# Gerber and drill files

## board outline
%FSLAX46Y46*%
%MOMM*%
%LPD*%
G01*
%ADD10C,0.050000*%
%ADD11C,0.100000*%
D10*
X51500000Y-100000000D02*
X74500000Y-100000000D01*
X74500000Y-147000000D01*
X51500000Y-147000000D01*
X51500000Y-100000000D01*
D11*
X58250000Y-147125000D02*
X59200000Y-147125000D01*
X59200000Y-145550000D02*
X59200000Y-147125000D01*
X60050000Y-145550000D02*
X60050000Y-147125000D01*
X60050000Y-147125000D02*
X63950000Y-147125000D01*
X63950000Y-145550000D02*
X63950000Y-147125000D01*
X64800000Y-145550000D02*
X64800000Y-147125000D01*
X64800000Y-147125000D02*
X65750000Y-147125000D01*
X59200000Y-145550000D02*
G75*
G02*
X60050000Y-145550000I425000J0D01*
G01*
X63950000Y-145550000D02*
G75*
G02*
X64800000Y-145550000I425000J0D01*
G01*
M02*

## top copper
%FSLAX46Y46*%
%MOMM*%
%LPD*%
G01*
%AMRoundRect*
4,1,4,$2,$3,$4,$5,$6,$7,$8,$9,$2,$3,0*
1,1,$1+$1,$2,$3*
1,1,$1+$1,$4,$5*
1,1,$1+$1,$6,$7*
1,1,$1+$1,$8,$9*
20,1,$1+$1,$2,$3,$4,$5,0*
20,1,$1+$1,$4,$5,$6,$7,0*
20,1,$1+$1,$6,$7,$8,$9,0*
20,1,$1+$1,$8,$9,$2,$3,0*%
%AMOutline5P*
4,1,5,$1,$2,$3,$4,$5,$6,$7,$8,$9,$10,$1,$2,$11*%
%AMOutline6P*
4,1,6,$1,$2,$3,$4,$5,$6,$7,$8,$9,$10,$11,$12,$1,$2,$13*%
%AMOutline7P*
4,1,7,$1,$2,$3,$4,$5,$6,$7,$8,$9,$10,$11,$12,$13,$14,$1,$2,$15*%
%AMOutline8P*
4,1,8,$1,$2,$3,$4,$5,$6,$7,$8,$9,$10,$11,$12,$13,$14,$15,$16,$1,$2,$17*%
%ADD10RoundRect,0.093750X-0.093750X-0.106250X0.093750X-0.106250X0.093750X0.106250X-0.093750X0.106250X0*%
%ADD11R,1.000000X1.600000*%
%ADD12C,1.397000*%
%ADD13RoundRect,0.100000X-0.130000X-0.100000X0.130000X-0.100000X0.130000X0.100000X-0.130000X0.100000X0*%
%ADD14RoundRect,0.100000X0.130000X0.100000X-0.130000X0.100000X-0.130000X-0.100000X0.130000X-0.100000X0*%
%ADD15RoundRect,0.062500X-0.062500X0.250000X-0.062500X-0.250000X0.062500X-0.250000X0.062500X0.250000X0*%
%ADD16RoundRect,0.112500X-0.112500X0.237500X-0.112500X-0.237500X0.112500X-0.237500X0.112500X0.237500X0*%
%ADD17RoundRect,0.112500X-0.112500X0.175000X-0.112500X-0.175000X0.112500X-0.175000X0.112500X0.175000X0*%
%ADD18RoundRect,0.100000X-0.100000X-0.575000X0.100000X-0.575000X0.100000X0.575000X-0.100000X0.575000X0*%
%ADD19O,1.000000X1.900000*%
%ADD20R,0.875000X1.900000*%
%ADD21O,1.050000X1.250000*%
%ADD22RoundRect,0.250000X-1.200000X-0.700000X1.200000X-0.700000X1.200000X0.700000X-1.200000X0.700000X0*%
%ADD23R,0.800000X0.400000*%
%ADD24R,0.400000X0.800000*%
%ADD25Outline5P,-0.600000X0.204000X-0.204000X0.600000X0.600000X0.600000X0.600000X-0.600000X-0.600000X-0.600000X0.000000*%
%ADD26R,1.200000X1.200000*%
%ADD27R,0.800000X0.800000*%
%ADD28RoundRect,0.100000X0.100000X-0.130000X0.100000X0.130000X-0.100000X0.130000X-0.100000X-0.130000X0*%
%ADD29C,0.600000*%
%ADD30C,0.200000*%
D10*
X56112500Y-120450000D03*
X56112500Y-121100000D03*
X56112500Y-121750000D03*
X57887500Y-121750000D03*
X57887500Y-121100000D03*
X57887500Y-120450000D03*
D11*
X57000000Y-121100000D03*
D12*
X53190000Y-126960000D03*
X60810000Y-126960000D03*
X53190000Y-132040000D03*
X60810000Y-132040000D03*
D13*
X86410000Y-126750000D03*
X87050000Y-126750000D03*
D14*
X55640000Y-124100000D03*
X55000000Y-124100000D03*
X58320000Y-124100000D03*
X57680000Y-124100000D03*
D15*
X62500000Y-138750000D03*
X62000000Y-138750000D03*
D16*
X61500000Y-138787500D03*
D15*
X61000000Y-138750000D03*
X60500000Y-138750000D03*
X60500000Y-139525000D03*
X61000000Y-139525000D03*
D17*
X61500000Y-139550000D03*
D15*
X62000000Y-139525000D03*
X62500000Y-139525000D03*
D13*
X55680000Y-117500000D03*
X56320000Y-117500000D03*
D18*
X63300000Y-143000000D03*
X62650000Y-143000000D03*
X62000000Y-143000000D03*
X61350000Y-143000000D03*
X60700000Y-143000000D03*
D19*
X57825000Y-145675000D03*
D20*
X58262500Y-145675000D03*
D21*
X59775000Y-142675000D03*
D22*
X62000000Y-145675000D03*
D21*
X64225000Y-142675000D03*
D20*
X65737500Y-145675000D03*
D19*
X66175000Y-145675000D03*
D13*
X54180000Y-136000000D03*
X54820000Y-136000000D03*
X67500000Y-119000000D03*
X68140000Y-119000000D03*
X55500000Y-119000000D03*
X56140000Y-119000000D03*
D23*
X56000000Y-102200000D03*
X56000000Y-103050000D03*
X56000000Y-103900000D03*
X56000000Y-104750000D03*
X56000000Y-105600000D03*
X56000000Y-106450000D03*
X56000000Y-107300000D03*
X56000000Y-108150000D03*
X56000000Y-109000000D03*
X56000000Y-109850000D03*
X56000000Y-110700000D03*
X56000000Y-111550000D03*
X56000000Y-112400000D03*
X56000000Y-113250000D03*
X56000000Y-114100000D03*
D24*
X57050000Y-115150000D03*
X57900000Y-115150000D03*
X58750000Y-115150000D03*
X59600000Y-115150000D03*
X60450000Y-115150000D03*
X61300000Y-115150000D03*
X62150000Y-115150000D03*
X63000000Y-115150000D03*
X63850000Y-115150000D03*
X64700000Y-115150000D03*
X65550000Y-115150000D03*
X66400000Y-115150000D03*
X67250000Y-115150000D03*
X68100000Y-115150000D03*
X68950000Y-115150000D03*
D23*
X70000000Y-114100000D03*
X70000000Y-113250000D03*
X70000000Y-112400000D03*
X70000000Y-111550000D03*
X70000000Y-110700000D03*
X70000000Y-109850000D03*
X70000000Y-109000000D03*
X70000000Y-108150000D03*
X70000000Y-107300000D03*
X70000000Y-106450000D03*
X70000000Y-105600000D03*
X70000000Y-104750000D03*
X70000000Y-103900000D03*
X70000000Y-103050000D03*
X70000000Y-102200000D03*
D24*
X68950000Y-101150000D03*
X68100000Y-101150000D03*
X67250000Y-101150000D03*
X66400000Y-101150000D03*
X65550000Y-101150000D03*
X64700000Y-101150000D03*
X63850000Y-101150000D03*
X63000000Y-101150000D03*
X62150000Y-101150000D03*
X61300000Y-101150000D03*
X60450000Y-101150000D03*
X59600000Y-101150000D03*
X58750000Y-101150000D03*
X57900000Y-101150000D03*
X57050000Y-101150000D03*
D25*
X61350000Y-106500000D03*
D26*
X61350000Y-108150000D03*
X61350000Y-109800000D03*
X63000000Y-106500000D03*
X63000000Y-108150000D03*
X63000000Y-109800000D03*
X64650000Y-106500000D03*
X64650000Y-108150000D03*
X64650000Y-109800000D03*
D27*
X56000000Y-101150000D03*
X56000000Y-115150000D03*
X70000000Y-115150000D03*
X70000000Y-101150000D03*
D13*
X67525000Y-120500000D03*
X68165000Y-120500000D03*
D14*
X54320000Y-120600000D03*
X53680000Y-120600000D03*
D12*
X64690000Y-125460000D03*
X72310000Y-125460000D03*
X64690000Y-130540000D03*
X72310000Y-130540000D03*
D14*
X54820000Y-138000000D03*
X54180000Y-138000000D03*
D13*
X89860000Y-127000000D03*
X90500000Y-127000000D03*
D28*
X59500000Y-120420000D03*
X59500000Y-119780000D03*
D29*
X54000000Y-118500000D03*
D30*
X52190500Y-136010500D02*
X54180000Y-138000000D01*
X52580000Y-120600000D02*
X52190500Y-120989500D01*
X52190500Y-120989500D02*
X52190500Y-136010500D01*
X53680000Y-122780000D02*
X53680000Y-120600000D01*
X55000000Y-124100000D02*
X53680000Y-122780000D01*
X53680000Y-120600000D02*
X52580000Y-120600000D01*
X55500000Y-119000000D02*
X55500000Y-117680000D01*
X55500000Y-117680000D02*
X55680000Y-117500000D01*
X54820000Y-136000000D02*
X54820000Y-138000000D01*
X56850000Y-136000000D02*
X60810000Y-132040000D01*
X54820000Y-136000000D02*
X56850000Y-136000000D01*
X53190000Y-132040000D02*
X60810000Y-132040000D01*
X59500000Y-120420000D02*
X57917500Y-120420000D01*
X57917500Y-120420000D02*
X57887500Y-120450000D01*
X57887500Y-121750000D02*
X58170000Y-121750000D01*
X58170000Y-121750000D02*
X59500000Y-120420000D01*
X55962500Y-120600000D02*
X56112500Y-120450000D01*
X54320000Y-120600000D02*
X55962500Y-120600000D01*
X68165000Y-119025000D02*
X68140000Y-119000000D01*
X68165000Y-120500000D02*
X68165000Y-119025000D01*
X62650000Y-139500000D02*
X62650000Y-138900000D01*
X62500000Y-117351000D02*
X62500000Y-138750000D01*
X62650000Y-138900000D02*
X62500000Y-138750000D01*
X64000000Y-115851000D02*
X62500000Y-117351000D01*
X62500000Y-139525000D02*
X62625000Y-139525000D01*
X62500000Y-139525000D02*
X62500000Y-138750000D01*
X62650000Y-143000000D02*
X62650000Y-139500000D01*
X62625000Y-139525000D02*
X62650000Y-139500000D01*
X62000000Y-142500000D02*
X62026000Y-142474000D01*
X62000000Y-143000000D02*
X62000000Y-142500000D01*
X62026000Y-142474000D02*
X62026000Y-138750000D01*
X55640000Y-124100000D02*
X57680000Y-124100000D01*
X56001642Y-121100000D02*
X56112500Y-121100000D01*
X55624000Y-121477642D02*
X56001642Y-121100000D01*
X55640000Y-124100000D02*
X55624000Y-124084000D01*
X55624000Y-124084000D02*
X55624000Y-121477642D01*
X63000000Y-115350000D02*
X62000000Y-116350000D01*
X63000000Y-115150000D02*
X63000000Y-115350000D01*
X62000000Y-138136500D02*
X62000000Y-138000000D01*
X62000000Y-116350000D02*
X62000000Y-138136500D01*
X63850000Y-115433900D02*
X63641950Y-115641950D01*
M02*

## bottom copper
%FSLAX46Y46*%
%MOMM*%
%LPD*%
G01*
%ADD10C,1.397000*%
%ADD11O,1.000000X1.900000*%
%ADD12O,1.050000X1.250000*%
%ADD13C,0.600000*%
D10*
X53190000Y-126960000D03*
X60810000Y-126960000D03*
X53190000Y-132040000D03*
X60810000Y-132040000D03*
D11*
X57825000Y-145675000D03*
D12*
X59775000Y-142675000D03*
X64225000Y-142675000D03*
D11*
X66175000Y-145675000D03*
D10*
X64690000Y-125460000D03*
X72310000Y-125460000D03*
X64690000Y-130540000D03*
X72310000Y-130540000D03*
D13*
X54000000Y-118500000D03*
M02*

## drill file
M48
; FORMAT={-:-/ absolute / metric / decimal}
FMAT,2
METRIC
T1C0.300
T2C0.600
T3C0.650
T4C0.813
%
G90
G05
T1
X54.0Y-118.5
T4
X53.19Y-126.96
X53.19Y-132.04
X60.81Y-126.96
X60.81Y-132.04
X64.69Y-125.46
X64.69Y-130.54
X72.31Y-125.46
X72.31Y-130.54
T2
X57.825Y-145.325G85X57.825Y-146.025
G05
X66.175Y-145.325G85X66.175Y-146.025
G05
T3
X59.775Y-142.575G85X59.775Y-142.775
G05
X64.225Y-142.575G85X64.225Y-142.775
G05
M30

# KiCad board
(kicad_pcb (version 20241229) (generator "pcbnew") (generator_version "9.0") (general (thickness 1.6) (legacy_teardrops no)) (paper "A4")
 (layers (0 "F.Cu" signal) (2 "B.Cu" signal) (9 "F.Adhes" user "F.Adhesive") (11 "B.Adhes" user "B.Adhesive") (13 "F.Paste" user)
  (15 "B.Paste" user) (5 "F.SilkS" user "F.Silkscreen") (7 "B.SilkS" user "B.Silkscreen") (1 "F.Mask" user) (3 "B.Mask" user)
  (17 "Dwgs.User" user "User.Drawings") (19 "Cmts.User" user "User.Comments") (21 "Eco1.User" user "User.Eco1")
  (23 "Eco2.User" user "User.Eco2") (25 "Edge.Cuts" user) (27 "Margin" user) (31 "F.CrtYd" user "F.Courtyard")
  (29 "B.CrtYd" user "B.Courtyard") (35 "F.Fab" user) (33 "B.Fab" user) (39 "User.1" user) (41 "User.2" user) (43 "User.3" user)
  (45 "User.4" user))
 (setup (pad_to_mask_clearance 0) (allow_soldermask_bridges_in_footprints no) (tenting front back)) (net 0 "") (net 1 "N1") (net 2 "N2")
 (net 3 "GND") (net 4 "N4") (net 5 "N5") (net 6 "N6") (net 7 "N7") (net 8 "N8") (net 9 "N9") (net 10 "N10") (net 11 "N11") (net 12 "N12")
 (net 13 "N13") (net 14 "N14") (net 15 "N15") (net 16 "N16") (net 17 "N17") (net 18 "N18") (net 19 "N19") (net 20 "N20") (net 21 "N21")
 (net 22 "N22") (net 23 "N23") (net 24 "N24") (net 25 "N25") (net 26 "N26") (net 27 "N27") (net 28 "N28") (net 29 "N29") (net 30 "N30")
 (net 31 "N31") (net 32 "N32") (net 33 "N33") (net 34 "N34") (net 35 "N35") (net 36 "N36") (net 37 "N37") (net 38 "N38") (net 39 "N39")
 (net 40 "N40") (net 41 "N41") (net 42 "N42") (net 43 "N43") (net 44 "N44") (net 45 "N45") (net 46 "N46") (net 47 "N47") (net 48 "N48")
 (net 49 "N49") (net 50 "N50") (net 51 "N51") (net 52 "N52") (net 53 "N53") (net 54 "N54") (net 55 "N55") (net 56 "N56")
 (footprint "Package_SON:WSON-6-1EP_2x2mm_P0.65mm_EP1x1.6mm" (layer "F.Cu") (at 57 121.1)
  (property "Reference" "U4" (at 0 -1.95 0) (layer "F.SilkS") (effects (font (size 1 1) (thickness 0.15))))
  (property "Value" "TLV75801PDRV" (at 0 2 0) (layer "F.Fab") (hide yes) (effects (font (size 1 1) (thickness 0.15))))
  (pad "" smd roundrect (at 0 -0.4) (size 0.81 0.64) (layers "F.Paste") (roundrect_rratio 0.25))
  (pad "" smd roundrect (at 0 0.4) (size 0.81 0.64) (layers "F.Paste") (roundrect_rratio 0.25))
  (pad "1" smd roundrect (at -0.8875 -0.65) (size 0.375 0.4) (layers "F.Cu" "F.Mask" "F.Paste") (roundrect_rratio 0.25) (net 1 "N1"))
  (pad "2" smd roundrect (at -0.8875 0) (size 0.375 0.4) (layers "F.Cu" "F.Mask" "F.Paste") (roundrect_rratio 0.25) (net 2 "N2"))
  (pad "3" smd roundrect (at -0.8875 0.65) (size 0.375 0.4) (layers "F.Cu" "F.Mask" "F.Paste") (roundrect_rratio 0.25) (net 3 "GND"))
  (pad "4" smd roundrect (at 0.8875 0.65) (size 0.375 0.4) (layers "F.Cu" "F.Mask" "F.Paste") (roundrect_rratio 0.25) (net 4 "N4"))
  (pad "5" smd roundrect (at 0.8875 0) (size 0.375 0.4) (layers "F.Cu" "F.Mask" "F.Paste") (roundrect_rratio 0.25) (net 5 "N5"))
  (pad "6" smd roundrect (at 0.8875 -0.65) (size 0.375 0.4) (layers "F.Cu" "F.Mask" "F.Paste") (roundrect_rratio 0.25) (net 4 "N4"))
  (pad "7" smd rect (at 0 0) (size 1 1.6) (layers "F.Cu" "F.Mask") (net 3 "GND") (zone_connect 2)))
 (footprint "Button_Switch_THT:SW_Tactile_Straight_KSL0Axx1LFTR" (layer "F.Cu") (at 53.19 126.96)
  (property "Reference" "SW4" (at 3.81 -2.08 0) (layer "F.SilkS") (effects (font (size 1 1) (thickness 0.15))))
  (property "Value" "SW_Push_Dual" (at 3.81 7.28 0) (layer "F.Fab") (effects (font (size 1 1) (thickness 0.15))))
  (pad "1" thru_hole circle (at 0 0) (size 1.397 1.397) (drill 0.8128) (layers "*.Cu" "*.Mask") (remove_unused_layers no) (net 3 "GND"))
  (pad "1" thru_hole circle (at 7.62 0) (size 1.397 1.397) (drill 0.8128) (layers "*.Cu" "*.Mask") (remove_unused_layers no) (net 3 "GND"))
  (pad "2" thru_hole circle (at 0 5.08) (size 1.397 1.397) (drill 0.8128) (layers "*.Cu" "*.Mask") (remove_unused_layers no) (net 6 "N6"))
  (pad "2" thru_hole circle (at 7.62 5.08) (size 1.397 1.397) (drill 0.8128) (layers "*.Cu" "*.Mask") (remove_unused_layers no) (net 6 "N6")))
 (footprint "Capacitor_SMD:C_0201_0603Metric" (layer "F.Cu") (at 86.73 126.75)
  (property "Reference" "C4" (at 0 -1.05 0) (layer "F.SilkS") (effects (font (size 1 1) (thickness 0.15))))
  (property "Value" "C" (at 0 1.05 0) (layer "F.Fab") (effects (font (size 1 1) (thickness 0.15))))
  (pad "" smd roundrect (at -0.345 0) (size 0.318 0.36) (layers "F.Paste") (roundrect_rratio 0.25))
  (pad "" smd roundrect (at 0.345 0) (size 0.318 0.36) (layers "F.Paste") (roundrect_rratio 0.25))
  (pad "1" smd roundrect (at -0.32 0) (size 0.46 0.4) (layers "F.Cu" "F.Mask") (roundrect_rratio 0.25) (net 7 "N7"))
  (pad "2" smd roundrect (at 0.32 0) (size 0.46 0.4) (layers "F.Cu" "F.Mask") (roundrect_rratio 0.25) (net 3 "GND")))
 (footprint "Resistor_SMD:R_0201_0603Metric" (layer "F.Cu") (at 55.32 124.1 180)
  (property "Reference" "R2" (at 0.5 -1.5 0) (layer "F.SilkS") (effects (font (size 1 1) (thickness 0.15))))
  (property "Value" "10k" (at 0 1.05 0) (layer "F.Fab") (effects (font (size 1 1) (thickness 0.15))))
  (pad "" smd roundrect (at -0.345 0 180) (size 0.318 0.36) (layers "F.Paste") (roundrect_rratio 0.25))
  (pad "" smd roundrect (at 0.345 0 180) (size 0.318 0.36) (layers "F.Paste") (roundrect_rratio 0.25))
  (pad "1" smd roundrect (at -0.32 0 180) (size 0.46 0.4) (layers "F.Cu" "F.Mask") (roundrect_rratio 0.25) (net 2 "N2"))
  (pad "2" smd roundrect (at 0.32 0 180) (size 0.46 0.4) (layers "F.Cu" "F.Mask") (roundrect_rratio 0.25) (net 3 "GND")))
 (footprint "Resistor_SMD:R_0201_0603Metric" (layer "F.Cu") (at 58 124.1 180)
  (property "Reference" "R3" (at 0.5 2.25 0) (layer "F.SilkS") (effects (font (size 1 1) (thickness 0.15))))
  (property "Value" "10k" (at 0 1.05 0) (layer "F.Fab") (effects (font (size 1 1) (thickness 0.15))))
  (pad "" smd roundrect (at -0.345 0 180) (size 0.318 0.36) (layers "F.Paste") (roundrect_rratio 0.25))
  (pad "" smd roundrect (at 0.345 0 180) (size 0.318 0.36) (layers "F.Paste") (roundrect_rratio 0.25))
  (pad "1" smd roundrect (at -0.32 0 180) (size 0.46 0.4) (layers "F.Cu" "F.Mask") (roundrect_rratio 0.25) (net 1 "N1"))
  (pad "2" smd roundrect (at 0.32 0 180) (size 0.46 0.4) (layers "F.Cu" "F.Mask") (roundrect_rratio 0.25) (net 2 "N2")))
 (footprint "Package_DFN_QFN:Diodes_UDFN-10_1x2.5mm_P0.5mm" (layer "F.Cu") (at 61.5 139.1375 -90)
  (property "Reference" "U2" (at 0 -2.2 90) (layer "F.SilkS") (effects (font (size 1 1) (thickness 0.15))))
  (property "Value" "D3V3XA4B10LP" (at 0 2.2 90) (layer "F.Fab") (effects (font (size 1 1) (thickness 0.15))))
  (pad "1" smd roundrect (at -0.3875 -1 270) (size 0.625 0.25) (layers "F.Cu" "F.Mask" "F.Paste") (roundrect_rratio 0.25) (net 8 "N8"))
  (pad "2" smd roundrect (at -0.3875 -0.5 270) (size 0.625 0.25) (layers "F.Cu" "F.Mask" "F.Paste") (roundrect_rratio 0.25) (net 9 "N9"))
  (pad "3" smd roundrect (at -0.35 0 270) (size 0.7 0.45) (layers "F.Cu" "F.Mask" "F.Paste") (roundrect_rratio 0.25) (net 3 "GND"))
  (pad "4" smd roundrect (at -0.3875 0.5 270) (size 0.625 0.25) (layers "F.Cu" "F.Mask" "F.Paste") (roundrect_rratio 0.25) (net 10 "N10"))
  (pad "5" smd roundrect (at -0.3875 1 270) (size 0.625 0.25) (layers "F.Cu" "F.Mask" "F.Paste") (roundrect_rratio 0.25) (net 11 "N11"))
  (pad "6" smd roundrect (at 0.3875 1 270) (size 0.625 0.25) (layers "F.Cu" "F.Mask" "F.Paste") (roundrect_rratio 0.25) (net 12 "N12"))
  (pad "7" smd roundrect (at 0.3875 0.5 270) (size 0.625 0.25) (layers "F.Cu" "F.Mask" "F.Paste") (roundrect_rratio 0.25) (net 10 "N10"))
  (pad "8" smd roundrect (at 0.4125 0 270) (size 0.575 0.45) (layers "F.Cu" "F.Mask" "F.Paste") (roundrect_rratio 0.25) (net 3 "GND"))
  (pad "9" smd roundrect (at 0.3875 -0.5 270) (size 0.625 0.25) (layers "F.Cu" "F.Mask" "F.Paste") (roundrect_rratio 0.25) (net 9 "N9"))
  (pad "10" smd roundrect (at 0.3875 -1 270) (size 0.625 0.25) (layers "F.Cu" "F.Mask" "F.Paste") (roundrect_rratio 0.25) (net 8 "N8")))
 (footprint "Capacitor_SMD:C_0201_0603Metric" (layer "F.Cu") (at 56 117.5)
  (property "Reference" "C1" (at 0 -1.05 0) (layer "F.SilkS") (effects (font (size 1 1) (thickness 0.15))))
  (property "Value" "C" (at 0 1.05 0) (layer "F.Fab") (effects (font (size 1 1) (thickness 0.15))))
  (pad "" smd roundrect (at -0.345 0) (size 0.318 0.36) (layers "F.Paste") (roundrect_rratio 0.25))
  (pad "" smd roundrect (at 0.345 0) (size 0.318 0.36) (layers "F.Paste") (roundrect_rratio 0.25))
  (pad "1" smd roundrect (at -0.32 0) (size 0.46 0.4) (layers "F.Cu" "F.Mask") (roundrect_rratio 0.25) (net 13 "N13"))
  (pad "2" smd roundrect (at 0.32 0) (size 0.46 0.4) (layers "F.Cu" "F.Mask") (roundrect_rratio 0.25) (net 3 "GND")))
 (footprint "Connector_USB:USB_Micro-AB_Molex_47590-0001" (layer "F.Cu") (at 62 146.025)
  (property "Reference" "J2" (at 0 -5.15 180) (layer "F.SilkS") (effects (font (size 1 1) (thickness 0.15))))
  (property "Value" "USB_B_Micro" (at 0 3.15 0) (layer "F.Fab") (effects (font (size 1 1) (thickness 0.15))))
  (fp_line (start -3.75 1.1) (end -2.8 1.1) (stroke (width 0.1) (type solid)) (layer "Edge.Cuts"))
  (fp_line (start -2.8 -0.475) (end -2.8 1.1) (stroke (width 0.1) (type solid)) (layer "Edge.Cuts"))
  (fp_line (start -1.95 -0.475) (end -1.95 1.1) (stroke (width 0.1) (type solid)) (layer "Edge.Cuts"))
  (fp_line (start -1.95 1.1) (end 1.95 1.1) (stroke (width 0.1) (type solid)) (layer "Edge.Cuts"))
  (fp_line (start 1.95 -0.475) (end 1.95 1.1) (stroke (width 0.1) (type solid)) (layer "Edge.Cuts"))
  (fp_line (start 2.8 -0.475) (end 2.8 1.1) (stroke (width 0.1) (type solid)) (layer "Edge.Cuts"))
  (fp_line (start 2.8 1.1) (end 3.75 1.1) (stroke (width 0.1) (type solid)) (layer "Edge.Cuts"))
  (fp_arc (start -2.8 -0.475) (mid -2.375 -0.9) (end -1.95 -0.475) (stroke (width 0.1) (type solid)) (layer "Edge.Cuts"))
  (fp_arc (start 1.95 -0.475) (mid 2.375 -0.9) (end 2.8 -0.475) (stroke (width 0.1) (type solid)) (layer "Edge.Cuts"))
  (pad "" smd rect (at -3.5 -0.35) (size 0.3 0.85) (layers "F.Paste"))
  (pad "" smd rect (at 3.5 -0.35) (size 0.3 0.85) (layers "F.Paste"))
  (pad "1" smd roundrect (at 1.3 -3.025) (size 0.4 1.35) (layers "F.Cu" "F.Mask" "F.Paste") (roundrect_rratio 0.25) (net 10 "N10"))
  (pad "2" smd roundrect (at 0.65 -3.025) (size 0.4 1.35) (layers "F.Cu" "F.Mask" "F.Paste") (roundrect_rratio 0.25) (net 8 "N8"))
  (pad "3" smd roundrect (at 0 -3.025) (size 0.4 1.35) (layers "F.Cu" "F.Mask" "F.Paste") (roundrect_rratio 0.25) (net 9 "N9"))
  (pad "4" smd roundrect (at -0.65 -3.025) (size 0.4 1.35) (layers "F.Cu" "F.Mask" "F.Paste") (roundrect_rratio 0.25) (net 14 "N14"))
  (pad "5" smd roundrect (at -1.3 -3.025) (size 0.4 1.35) (layers "F.Cu" "F.Mask" "F.Paste") (roundrect_rratio 0.25) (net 3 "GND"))
  (pad "6" thru_hole oval (at -4.175 -0.35) (size 1 1.9) (drill oval 0.6 1.3) (layers "*.Cu" "*.Mask") (remove_unused_layers no)
   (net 3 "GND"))
  (pad "6" smd rect (at -3.7375 -0.35) (size 0.875 1.9) (layers "F.Cu" "F.Mask") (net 3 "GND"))
  (pad "6" thru_hole oval (at -2.225 -3.35) (size 1.05 1.25) (drill oval 0.65 0.85) (layers "*.Cu" "*.Mask") (remove_unused_layers no)
   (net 3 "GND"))
  (pad "6" smd roundrect (at 0 -0.35) (size 2.9 1.9) (layers "F.Cu" "F.Mask" "F.Paste") (roundrect_rratio 0.1315789474) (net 3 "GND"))
  (pad "6" thru_hole oval (at 2.225 -3.35) (size 1.05 1.25) (drill oval 0.65 0.85) (layers "*.Cu" "*.Mask") (remove_unused_layers no)
   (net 3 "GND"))
  (pad "6" smd rect (at 3.7375 -0.35) (size 0.875 1.9) (layers "F.Cu" "F.Mask") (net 3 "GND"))
  (pad "6" thru_hole oval (at 4.175 -0.35) (size 1 1.9) (drill oval 0.6 1.3) (layers "*.Cu" "*.Mask") (remove_unused_layers no)
   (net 3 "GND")))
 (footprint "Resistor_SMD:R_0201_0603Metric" (layer "F.Cu") (at 54.5 136)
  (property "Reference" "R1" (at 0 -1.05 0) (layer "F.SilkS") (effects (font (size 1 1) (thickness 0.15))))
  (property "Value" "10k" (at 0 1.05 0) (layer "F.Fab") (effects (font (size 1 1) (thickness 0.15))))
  (pad "" smd roundrect (at -0.345 0) (size 0.318 0.36) (layers "F.Paste") (roundrect_rratio 0.25))
  (pad "" smd roundrect (at 0.345 0) (size 0.318 0.36) (layers "F.Paste") (roundrect_rratio 0.25))
  (pad "1" smd roundrect (at -0.32 0) (size 0.46 0.4) (layers "F.Cu" "F.Mask") (roundrect_rratio 0.25) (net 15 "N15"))
  (pad "2" smd roundrect (at 0.32 0) (size 0.46 0.4) (layers "F.Cu" "F.Mask") (roundrect_rratio 0.25) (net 6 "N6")))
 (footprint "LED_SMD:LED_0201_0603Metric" (layer "F.Cu") (at 67.82 119)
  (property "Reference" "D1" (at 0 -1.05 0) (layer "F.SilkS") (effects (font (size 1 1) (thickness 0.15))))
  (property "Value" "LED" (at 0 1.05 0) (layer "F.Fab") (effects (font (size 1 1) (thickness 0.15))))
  (pad "" smd roundrect (at -0.345 0) (size 0.318 0.36) (layers "F.Paste") (roundrect_rratio 0.25))
  (pad "" smd roundrect (at 0.345 0) (size 0.318 0.36) (layers "F.Paste") (roundrect_rratio 0.25))
  (pad "1" smd roundrect (at -0.32 0) (size 0.46 0.4) (layers "F.Cu" "F.Mask") (roundrect_rratio 0.25) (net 3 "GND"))
  (pad "2" smd roundrect (at 0.32 0) (size 0.46 0.4) (layers "F.Cu" "F.Mask") (roundrect_rratio 0.25) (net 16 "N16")))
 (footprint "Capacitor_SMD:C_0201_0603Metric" (layer "F.Cu") (at 55.82 119)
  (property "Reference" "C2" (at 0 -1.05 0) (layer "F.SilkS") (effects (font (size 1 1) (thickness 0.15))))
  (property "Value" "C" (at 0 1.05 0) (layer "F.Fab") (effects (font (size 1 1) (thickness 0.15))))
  (pad "" smd roundrect (at -0.345 0) (size 0.318 0.36) (layers "F.Paste") (roundrect_rratio 0.25))
  (pad "" smd roundrect (at 0.345 0) (size 0.318 0.36) (layers "F.Paste") (roundrect_rratio 0.25))
  (pad "1" smd roundrect (at -0.32 0) (size 0.46 0.4) (layers "F.Cu" "F.Mask") (roundrect_rratio 0.25) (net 13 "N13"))
  (pad "2" smd roundrect (at 0.32 0) (size 0.46 0.4) (layers "F.Cu" "F.Mask") (roundrect_rratio 0.25) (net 3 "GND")))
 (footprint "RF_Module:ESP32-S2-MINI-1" (layer "F.Cu") (at 63 105.6)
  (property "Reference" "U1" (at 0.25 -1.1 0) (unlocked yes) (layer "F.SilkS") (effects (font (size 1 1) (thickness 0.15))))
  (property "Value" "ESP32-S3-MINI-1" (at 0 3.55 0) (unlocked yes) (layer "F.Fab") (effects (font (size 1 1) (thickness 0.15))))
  (pad "1" smd rect (at -7 -3.4) (size 0.8 0.4) (layers "F.Cu" "F.Mask" "F.Paste") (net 3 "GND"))
  (pad "2" smd rect (at -7 -2.55) (size 0.8 0.4) (layers "F.Cu" "F.Mask" "F.Paste") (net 3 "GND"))
  (pad "3" smd rect (at -7 -1.7) (size 0.8 0.4) (layers "F.Cu" "F.Mask" "F.Paste") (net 13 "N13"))
  (pad "4" smd rect (at -7 -0.85) (size 0.8 0.4) (layers "F.Cu" "F.Mask" "F.Paste") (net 7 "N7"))
  (pad "5" smd rect (at -7 0) (size 0.8 0.4) (layers "F.Cu" "F.Mask" "F.Paste") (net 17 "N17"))
  (pad "6" smd rect (at -7 0.85) (size 0.8 0.4) (layers "F.Cu" "F.Mask" "F.Paste") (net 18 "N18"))
  (pad "7" smd rect (at -7 1.7) (size 0.8 0.4) (layers "F.Cu" "F.Mask" "F.Paste") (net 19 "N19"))
  (pad "8" smd rect (at -7 2.55) (size 0.8 0.4) (layers "F.Cu" "F.Mask" "F.Paste") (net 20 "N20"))
  (pad "9" smd rect (at -7 3.4) (size 0.8 0.4) (layers "F.Cu" "F.Mask" "F.Paste") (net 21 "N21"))
  (pad "10" smd rect (at -7 4.25) (size 0.8 0.4) (layers "F.Cu" "F.Mask" "F.Paste") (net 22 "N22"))
  (pad "11" smd rect (at -7 5.1) (size 0.8 0.4) (layers "F.Cu" "F.Mask" "F.Paste") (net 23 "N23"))
  (pad "12" smd rect (at -7 5.95) (size 0.8 0.4) (layers "F.Cu" "F.Mask" "F.Paste") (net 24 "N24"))
  (pad "13" smd rect (at -7 6.8) (size 0.8 0.4) (layers "F.Cu" "F.Mask" "F.Paste") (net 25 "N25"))
  (pad "14" smd rect (at -7 7.65) (size 0.8 0.4) (layers "F.Cu" "F.Mask" "F.Paste") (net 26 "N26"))
  (pad "15" smd rect (at -7 8.5) (size 0.8 0.4) (layers "F.Cu" "F.Mask" "F.Paste") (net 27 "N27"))
  (pad "16" smd rect (at -5.95 9.55 90) (size 0.8 0.4) (layers "F.Cu" "F.Mask" "F.Paste") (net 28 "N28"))
  (pad "17" smd rect (at -5.1 9.55 90) (size 0.8 0.4) (layers "F.Cu" "F.Mask" "F.Paste") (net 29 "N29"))
  (pad "18" smd rect (at -4.25 9.55 90) (size 0.8 0.4) (layers "F.Cu" "F.Mask" "F.Paste") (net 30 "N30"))
  (pad "19" smd rect (at -3.4 9.55 90) (size 0.8 0.4) (layers "F.Cu" "F.Mask" "F.Paste") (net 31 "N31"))
  (pad "20" smd rect (at -2.55 9.55 90) (size 0.8 0.4) (layers "F.Cu" "F.Mask" "F.Paste") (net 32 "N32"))
  (pad "21" smd rect (at -1.7 9.55 90) (size 0.8 0.4) (layers "F.Cu" "F.Mask" "F.Paste") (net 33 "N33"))
  (pad "22" smd rect (at -0.85 9.55 90) (size 0.8 0.4) (layers "F.Cu" "F.Mask" "F.Paste") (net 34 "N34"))
  (pad "23" smd rect (at 0 9.55 90) (size 0.8 0.4) (layers "F.Cu" "F.Mask" "F.Paste") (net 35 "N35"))
  (pad "24" smd rect (at 0.85 9.55 90) (size 0.8 0.4) (layers "F.Cu" "F.Mask" "F.Paste") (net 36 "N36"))
  (pad "25" smd rect (at 1.7 9.55 90) (size 0.8 0.4) (layers "F.Cu" "F.Mask" "F.Paste") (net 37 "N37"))
  (pad "26" smd rect (at 2.55 9.55 90) (size 0.8 0.4) (layers "F.Cu" "F.Mask" "F.Paste") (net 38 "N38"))
  (pad "27" smd rect (at 3.4 9.55 90) (size 0.8 0.4) (layers "F.Cu" "F.Mask" "F.Paste") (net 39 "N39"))
  (pad "28" smd rect (at 4.25 9.55 90) (size 0.8 0.4) (layers "F.Cu" "F.Mask" "F.Paste") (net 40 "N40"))
  (pad "29" smd rect (at 5.1 9.55 90) (size 0.8 0.4) (layers "F.Cu" "F.Mask" "F.Paste") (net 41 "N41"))
  (pad "30" smd rect (at 5.95 9.55 90) (size 0.8 0.4) (layers "F.Cu" "F.Mask" "F.Paste") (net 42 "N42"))
  (pad "31" smd rect (at 7 8.5) (size 0.8 0.4) (layers "F.Cu" "F.Mask" "F.Paste") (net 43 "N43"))
  (pad "32" smd rect (at 7 7.65) (size 0.8 0.4) (layers "F.Cu" "F.Mask" "F.Paste") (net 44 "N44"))
  (pad "33" smd rect (at 7 6.8) (size 0.8 0.4) (layers "F.Cu" "F.Mask" "F.Paste") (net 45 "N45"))
  (pad "34" smd rect (at 7 5.95) (size 0.8 0.4) (layers "F.Cu" "F.Mask" "F.Paste") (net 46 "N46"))
  (pad "35" smd rect (at 7 5.1) (size 0.8 0.4) (layers "F.Cu" "F.Mask" "F.Paste") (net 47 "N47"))
  (pad "36" smd rect (at 7 4.25) (size 0.8 0.4) (layers "F.Cu" "F.Mask" "F.Paste") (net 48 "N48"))
  (pad "37" smd rect (at 7 3.4) (size 0.8 0.4) (layers "F.Cu" "F.Mask" "F.Paste") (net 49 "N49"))
  (pad "38" smd rect (at 7 2.55) (size 0.8 0.4) (layers "F.Cu" "F.Mask" "F.Paste") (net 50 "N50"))
  (pad "39" smd rect (at 7 1.7) (size 0.8 0.4) (layers "F.Cu" "F.Mask" "F.Paste") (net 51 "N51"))
  (pad "40" smd rect (at 7 0.85) (size 0.8 0.4) (layers "F.Cu" "F.Mask" "F.Paste") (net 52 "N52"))
  (pad "41" smd rect (at 7 0) (size 0.8 0.4) (layers "F.Cu" "F.Mask" "F.Paste") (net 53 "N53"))
  (pad "42" smd rect (at 7 -0.85) (size 0.8 0.4) (layers "F.Cu" "F.Mask" "F.Paste") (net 3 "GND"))
  (pad "43" smd rect (at 7 -1.7) (size 0.8 0.4) (layers "F.Cu" "F.Mask" "F.Paste") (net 3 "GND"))
  (pad "44" smd rect (at 7 -2.55) (size 0.8 0.4) (layers "F.Cu" "F.Mask" "F.Paste") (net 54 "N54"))
  (pad "45" smd rect (at 7 -3.4) (size 0.8 0.4) (layers "F.Cu" "F.Mask" "F.Paste") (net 6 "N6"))
  (pad "46" smd rect (at 5.95 -4.45 90) (size 0.8 0.4) (layers "F.Cu" "F.Mask" "F.Paste") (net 3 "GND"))
  (pad "47" smd rect (at 5.1 -4.45 90) (size 0.8 0.4) (layers "F.Cu" "F.Mask" "F.Paste") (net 3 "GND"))
  (pad "48" smd rect (at 4.25 -4.45 90) (size 0.8 0.4) (layers "F.Cu" "F.Mask" "F.Paste") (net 3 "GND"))
  (pad "49" smd rect (at 3.4 -4.45 90) (size 0.8 0.4) (layers "F.Cu" "F.Mask" "F.Paste") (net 3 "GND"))
  (pad "50" smd rect (at 2.55 -4.45 90) (size 0.8 0.4) (layers "F.Cu" "F.Mask" "F.Paste") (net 3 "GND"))
  (pad "51" smd rect (at 1.7 -4.45 90) (size 0.8 0.4) (layers "F.Cu" "F.Mask" "F.Paste") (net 3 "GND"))
  (pad "52" smd rect (at 0.85 -4.45 90) (size 0.8 0.4) (layers "F.Cu" "F.Mask" "F.Paste") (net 3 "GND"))
  (pad "53" smd rect (at 0 -4.45 90) (size 0.8 0.4) (layers "F.Cu" "F.Mask" "F.Paste") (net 3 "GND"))
  (pad "54" smd rect (at -0.85 -4.45 90) (size 0.8 0.4) (layers "F.Cu" "F.Mask" "F.Paste") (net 3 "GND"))
  (pad "55" smd rect (at -1.7 -4.45 90) (size 0.8 0.4) (layers "F.Cu" "F.Mask" "F.Paste") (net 3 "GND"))
  (pad "56" smd rect (at -2.55 -4.45 90) (size 0.8 0.4) (layers "F.Cu" "F.Mask" "F.Paste") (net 3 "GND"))
  (pad "57" smd rect (at -3.4 -4.45 90) (size 0.8 0.4) (layers "F.Cu" "F.Mask" "F.Paste") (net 3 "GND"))
  (pad "58" smd rect (at -4.25 -4.45 90) (size 0.8 0.4) (layers "F.Cu" "F.Mask" "F.Paste") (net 3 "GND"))
  (pad "59" smd rect (at -5.1 -4.45 90) (size 0.8 0.4) (layers "F.Cu" "F.Mask" "F.Paste") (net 3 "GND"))
  (pad "60" smd rect (at -5.95 -4.45 90) (size 0.8 0.4) (layers "F.Cu" "F.Mask" "F.Paste") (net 3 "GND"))
  (pad "61" smd roundrect (at -1.65 0.9) (size 1.2 1.2) (layers "F.Cu" "F.Mask" "F.Paste") (roundrect_rratio 0) (chamfer_ratio 0.33)
   (chamfer top_left) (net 3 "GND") (zone_connect 2))
  (pad "61" smd rect (at -1.65 2.55) (size 1.2 1.2) (layers "F.Cu" "F.Mask" "F.Paste") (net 3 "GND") (zone_connect 2))
  (pad "61" smd rect (at -1.65 4.2) (size 1.2 1.2) (layers "F.Cu" "F.Mask" "F.Paste") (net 3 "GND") (zone_connect 2))
  (pad "61" smd rect (at 0 0.9) (size 1.2 1.2) (layers "F.Cu" "F.Mask" "F.Paste") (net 3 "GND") (zone_connect 2))
  (pad "61" smd rect (at 0 2.55) (size 1.2 1.2) (layers "F.Cu" "F.Mask" "F.Paste") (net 3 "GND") (zone_connect 2))
  (pad "61" smd rect (at 0 4.2) (size 1.2 1.2) (layers "F.Cu" "F.Mask" "F.Paste") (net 3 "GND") (zone_connect 2))
  (pad "61" smd rect (at 1.65 0.9) (size 1.2 1.2) (layers "F.Cu" "F.Mask" "F.Paste") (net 3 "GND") (zone_connect 2))
  (pad "61" smd rect (at 1.65 2.55) (size 1.2 1.2) (layers "F.Cu" "F.Mask" "F.Paste") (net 3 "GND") (zone_connect 2))
  (pad "61" smd rect (at 1.65 4.2) (size 1.2 1.2) (layers "F.Cu" "F.Mask" "F.Paste") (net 3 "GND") (zone_connect 2))
  (pad "62" smd rect (at -7 -4.45) (size 0.8 0.8) (layers "F.Cu" "F.Mask" "F.Paste") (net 3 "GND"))
  (pad "63" smd rect (at -7 9.55) (size 0.8 0.8) (layers "F.Cu" "F.Mask" "F.Paste") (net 3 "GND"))
  (pad "64" smd rect (at 7 9.55) (size 0.8 0.8) (layers "F.Cu" "F.Mask" "F.Paste") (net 3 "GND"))
  (pad "65" smd rect (at 7 -4.45) (size 0.8 0.8) (layers "F.Cu" "F.Mask" "F.Paste") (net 3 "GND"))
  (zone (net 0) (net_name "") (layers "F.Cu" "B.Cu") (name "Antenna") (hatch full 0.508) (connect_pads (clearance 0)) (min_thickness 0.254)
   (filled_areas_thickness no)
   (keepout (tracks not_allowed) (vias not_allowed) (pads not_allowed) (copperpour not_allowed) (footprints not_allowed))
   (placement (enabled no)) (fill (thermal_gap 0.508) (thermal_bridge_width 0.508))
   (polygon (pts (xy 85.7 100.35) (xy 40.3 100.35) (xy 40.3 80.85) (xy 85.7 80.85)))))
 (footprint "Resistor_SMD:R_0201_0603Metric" (layer "F.Cu") (at 67.845 120.5)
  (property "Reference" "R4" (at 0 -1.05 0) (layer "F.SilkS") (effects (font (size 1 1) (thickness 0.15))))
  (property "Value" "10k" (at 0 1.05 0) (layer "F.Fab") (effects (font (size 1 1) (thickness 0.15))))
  (pad "" smd roundrect (at -0.345 0) (size 0.318 0.36) (layers "F.Paste") (roundrect_rratio 0.25))
  (pad "" smd roundrect (at 0.345 0) (size 0.318 0.36) (layers "F.Paste") (roundrect_rratio 0.25))
  (pad "1" smd roundrect (at -0.32 0) (size 0.46 0.4) (layers "F.Cu" "F.Mask") (roundrect_rratio 0.25) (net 1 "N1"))
  (pad "2" smd roundrect (at 0.32 0) (size 0.46 0.4) (layers "F.Cu" "F.Mask") (roundrect_rratio 0.25) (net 16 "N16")))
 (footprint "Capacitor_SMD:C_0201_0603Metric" (layer "F.Cu") (at 54 120.6 180)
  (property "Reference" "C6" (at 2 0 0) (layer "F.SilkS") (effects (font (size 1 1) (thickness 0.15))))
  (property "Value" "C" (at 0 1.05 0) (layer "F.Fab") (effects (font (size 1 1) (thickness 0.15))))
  (pad "" smd roundrect (at -0.345 0 180) (size 0.318 0.36) (layers "F.Paste") (roundrect_rratio 0.25))
  (pad "" smd roundrect (at 0.345 0 180) (size 0.318 0.36) (layers "F.Paste") (roundrect_rratio 0.25))
  (pad "1" smd roundrect (at -0.32 0 180) (size 0.46 0.4) (layers "F.Cu" "F.Mask") (roundrect_rratio 0.25) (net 1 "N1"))
  (pad "2" smd roundrect (at 0.32 0 180) (size 0.46 0.4) (layers "F.Cu" "F.Mask") (roundrect_rratio 0.25) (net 3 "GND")))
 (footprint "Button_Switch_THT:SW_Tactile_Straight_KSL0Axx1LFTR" (layer "F.Cu") (at 64.69 125.46)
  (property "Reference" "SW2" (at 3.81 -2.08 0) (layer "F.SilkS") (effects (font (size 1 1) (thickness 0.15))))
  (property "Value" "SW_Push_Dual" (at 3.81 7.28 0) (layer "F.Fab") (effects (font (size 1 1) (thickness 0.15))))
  (pad "1" thru_hole circle (at 0 0) (size 1.397 1.397) (drill 0.8128) (layers "*.Cu" "*.Mask") (remove_unused_layers no) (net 3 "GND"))
  (pad "1" thru_hole circle (at 7.62 0) (size 1.397 1.397) (drill 0.8128) (layers "*.Cu" "*.Mask") (remove_unused_layers no) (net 3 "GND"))
  (pad "2" thru_hole circle (at 0 5.08) (size 1.397 1.397) (drill 0.8128) (layers "*.Cu" "*.Mask") (remove_unused_layers no) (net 7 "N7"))
  (pad "2" thru_hole circle (at 7.62 5.08) (size 1.397 1.397) (drill 0.8128) (layers "*.Cu" "*.Mask") (remove_unused_layers no) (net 7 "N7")))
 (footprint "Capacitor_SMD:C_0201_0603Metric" (layer "F.Cu") (at 54.5 138 180)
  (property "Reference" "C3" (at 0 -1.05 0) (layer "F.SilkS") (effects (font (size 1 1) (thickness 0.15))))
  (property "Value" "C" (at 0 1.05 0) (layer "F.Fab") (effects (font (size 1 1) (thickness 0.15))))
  (pad "" smd roundrect (at -0.345 0 180) (size 0.318 0.36) (layers "F.Paste") (roundrect_rratio 0.25))
  (pad "" smd roundrect (at 0.345 0 180) (size 0.318 0.36) (layers "F.Paste") (roundrect_rratio 0.25))
  (pad "1" smd roundrect (at -0.32 0 180) (size 0.46 0.4) (layers "F.Cu" "F.Mask") (roundrect_rratio 0.25) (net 6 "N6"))
  (pad "2" smd roundrect (at 0.32 0 180) (size 0.46 0.4) (layers "F.Cu" "F.Mask") (roundrect_rratio 0.25) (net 3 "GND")))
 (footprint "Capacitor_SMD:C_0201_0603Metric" (layer "F.Cu") (at 90.18 127)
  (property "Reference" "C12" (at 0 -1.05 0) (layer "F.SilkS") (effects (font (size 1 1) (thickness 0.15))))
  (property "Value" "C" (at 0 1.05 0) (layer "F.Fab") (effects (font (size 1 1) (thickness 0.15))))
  (pad "" smd roundrect (at -0.345 0) (size 0.318 0.36) (layers "F.Paste") (roundrect_rratio 0.25))
  (pad "" smd roundrect (at 0.345 0) (size 0.318 0.36) (layers "F.Paste") (roundrect_rratio 0.25))
  (pad "1" smd roundrect (at -0.32 0) (size 0.46 0.4) (layers "F.Cu" "F.Mask") (roundrect_rratio 0.25) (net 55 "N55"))
  (pad "2" smd roundrect (at 0.32 0) (size 0.46 0.4) (layers "F.Cu" "F.Mask") (roundrect_rratio 0.25) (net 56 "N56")))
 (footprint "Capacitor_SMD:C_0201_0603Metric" (layer "F.Cu") (at 59.5 120.1 90)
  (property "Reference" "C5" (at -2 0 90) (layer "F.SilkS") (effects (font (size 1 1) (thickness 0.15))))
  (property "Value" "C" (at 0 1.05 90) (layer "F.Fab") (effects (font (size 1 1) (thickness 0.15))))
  (pad "" smd roundrect (at -0.345 0 90) (size 0.318 0.36) (layers "F.Paste") (roundrect_rratio 0.25))
  (pad "" smd roundrect (at 0.345 0 90) (size 0.318 0.36) (layers "F.Paste") (roundrect_rratio 0.25))
  (pad "1" smd roundrect (at -0.32 0 90) (size 0.46 0.4) (layers "F.Cu" "F.Mask") (roundrect_rratio 0.25) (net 4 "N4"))
  (pad "2" smd roundrect (at 0.32 0 90) (size 0.46 0.4) (layers "F.Cu" "F.Mask") (roundrect_rratio 0.25) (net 3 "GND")))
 (gr_rect (start 51.5 100) (end 74.5 147) (stroke (width 0.05) (type default)) (fill no) (layer "Edge.Cuts"))
 (via (at 54 118.5) (size 0.6) (drill 0.3) (layers "F.Cu" "B.Cu") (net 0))
 (segment (start 52.1905 136.0105) (end 54.18 138) (width 0.2) (layer "F.Cu") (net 3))
 (segment (start 52.58 120.6) (end 52.1905 120.9895) (width 0.2) (layer "F.Cu") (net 3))
 (segment (start 52.1905 120.9895) (end 52.1905 136.0105) (width 0.2) (layer "F.Cu") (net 3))
 (segment (start 53.68 122.78) (end 53.68 120.6) (width 0.2) (layer "F.Cu") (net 3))
 (segment (start 55 124.1) (end 53.68 122.78) (width 0.2) (layer "F.Cu") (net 3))
 (segment (start 53.68 120.6) (end 52.58 120.6) (width 0.2) (layer "F.Cu") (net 3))
 (segment (start 55.5 119) (end 55.5 117.68) (width 0.2) (layer "F.Cu") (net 13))
 (segment (start 55.5 117.68) (end 55.68 117.5) (width 0.2) (layer "F.Cu") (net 13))
 (segment (start 54.82 136) (end 54.82 138) (width 0.2) (layer "F.Cu") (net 6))
 (segment (start 56.85 136) (end 60.81 132.04) (width 0.2) (layer "F.Cu") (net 6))
 (segment (start 54.82 136) (end 56.85 136) (width 0.2) (layer "F.Cu") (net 6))
 (segment (start 53.19 132.04) (end 60.81 132.04) (width 0.2) (layer "F.Cu") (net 6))
 (segment (start 59.5 120.42) (end 57.9175 120.42) (width 0.2) (layer "F.Cu") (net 4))
 (segment (start 57.9175 120.42) (end 57.8875 120.45) (width 0.2) (layer "F.Cu") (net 4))
 (segment (start 57.8875 121.75) (end 58.17 121.75) (width 0.2) (layer "F.Cu") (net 4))
 (segment (start 58.17 121.75) (end 59.5 120.42) (width 0.2) (layer "F.Cu") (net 4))
 (segment (start 55.9625 120.6) (end 56.1125 120.45) (width 0.2) (layer "F.Cu") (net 1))
 (segment (start 54.32 120.6) (end 55.9625 120.6) (width 0.2) (layer "F.Cu") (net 1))
 (segment (start 68.165 119.025) (end 68.14 119) (width 0.2) (layer "F.Cu") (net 16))
 (segment (start 68.165 120.5) (end 68.165 119.025) (width 0.2) (layer "F.Cu") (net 16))
 (segment (start 62.65 139.5) (end 62.65 138.9) (width 0.2) (layer "F.Cu") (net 8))
 (segment (start 62.5 117.351) (end 62.5 138.75) (width 0.2) (layer "F.Cu") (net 8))
 (segment (start 62.65 138.9) (end 62.5 138.75) (width 0.2) (layer "F.Cu") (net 8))
 (segment (start 64 115.851) (end 62.5 117.351) (width 0.2) (layer "F.Cu") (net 8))
 (segment (start 62.5 139.525) (end 62.625 139.525) (width 0.2) (layer "F.Cu") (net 8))
 (segment (start 62.5 139.525) (end 62.5 138.75) (width 0.2) (layer "F.Cu") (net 8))
 (segment (start 62.65 143) (end 62.65 139.5) (width 0.2) (layer "F.Cu") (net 8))
 (segment (start 62.625 139.525) (end 62.65 139.5) (width 0.2) (layer "F.Cu") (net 8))
 (segment (start 62 142.5) (end 62.026 142.474) (width 0.2) (layer "F.Cu") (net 9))
 (segment (start 62 143) (end 62 142.5) (width 0.2) (layer "F.Cu") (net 9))
 (segment (start 62.026 142.474) (end 62.026 138.75) (width 0.2) (layer "F.Cu") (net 9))
 (segment (start 55.64 124.1) (end 57.68 124.1) (width 0.2) (layer "F.Cu") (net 2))
 (segment (start 56.001642 121.1) (end 56.1125 121.1) (width 0.2) (layer "F.Cu") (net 2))
 (segment (start 55.624 121.477642) (end 56.001642 121.1) (width 0.2) (layer "F.Cu") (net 2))
 (segment (start 55.64 124.1) (end 55.624 124.084) (width 0.2) (layer "F.Cu") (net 2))
 (segment (start 55.624 124.084) (end 55.624 121.477642) (width 0.2) (layer "F.Cu") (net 2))
 (segment (start 63 115.35) (end 62 116.35) (width 0.2) (layer "F.Cu") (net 35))
 (segment (start 63 115.15) (end 63 115.35) (width 0.2) (layer "F.Cu") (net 35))
 (segment (start 62 138.1365) (end 62 138) (width 0.2) (layer "F.Cu") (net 35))
 (segment (start 62 116.35) (end 62 138.1365) (width 0.2) (layer "F.Cu") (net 35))
 (segment (start 63.85 115.4339) (end 63.64195 115.64195) (width 0.2) (layer "F.Cu") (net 36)))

